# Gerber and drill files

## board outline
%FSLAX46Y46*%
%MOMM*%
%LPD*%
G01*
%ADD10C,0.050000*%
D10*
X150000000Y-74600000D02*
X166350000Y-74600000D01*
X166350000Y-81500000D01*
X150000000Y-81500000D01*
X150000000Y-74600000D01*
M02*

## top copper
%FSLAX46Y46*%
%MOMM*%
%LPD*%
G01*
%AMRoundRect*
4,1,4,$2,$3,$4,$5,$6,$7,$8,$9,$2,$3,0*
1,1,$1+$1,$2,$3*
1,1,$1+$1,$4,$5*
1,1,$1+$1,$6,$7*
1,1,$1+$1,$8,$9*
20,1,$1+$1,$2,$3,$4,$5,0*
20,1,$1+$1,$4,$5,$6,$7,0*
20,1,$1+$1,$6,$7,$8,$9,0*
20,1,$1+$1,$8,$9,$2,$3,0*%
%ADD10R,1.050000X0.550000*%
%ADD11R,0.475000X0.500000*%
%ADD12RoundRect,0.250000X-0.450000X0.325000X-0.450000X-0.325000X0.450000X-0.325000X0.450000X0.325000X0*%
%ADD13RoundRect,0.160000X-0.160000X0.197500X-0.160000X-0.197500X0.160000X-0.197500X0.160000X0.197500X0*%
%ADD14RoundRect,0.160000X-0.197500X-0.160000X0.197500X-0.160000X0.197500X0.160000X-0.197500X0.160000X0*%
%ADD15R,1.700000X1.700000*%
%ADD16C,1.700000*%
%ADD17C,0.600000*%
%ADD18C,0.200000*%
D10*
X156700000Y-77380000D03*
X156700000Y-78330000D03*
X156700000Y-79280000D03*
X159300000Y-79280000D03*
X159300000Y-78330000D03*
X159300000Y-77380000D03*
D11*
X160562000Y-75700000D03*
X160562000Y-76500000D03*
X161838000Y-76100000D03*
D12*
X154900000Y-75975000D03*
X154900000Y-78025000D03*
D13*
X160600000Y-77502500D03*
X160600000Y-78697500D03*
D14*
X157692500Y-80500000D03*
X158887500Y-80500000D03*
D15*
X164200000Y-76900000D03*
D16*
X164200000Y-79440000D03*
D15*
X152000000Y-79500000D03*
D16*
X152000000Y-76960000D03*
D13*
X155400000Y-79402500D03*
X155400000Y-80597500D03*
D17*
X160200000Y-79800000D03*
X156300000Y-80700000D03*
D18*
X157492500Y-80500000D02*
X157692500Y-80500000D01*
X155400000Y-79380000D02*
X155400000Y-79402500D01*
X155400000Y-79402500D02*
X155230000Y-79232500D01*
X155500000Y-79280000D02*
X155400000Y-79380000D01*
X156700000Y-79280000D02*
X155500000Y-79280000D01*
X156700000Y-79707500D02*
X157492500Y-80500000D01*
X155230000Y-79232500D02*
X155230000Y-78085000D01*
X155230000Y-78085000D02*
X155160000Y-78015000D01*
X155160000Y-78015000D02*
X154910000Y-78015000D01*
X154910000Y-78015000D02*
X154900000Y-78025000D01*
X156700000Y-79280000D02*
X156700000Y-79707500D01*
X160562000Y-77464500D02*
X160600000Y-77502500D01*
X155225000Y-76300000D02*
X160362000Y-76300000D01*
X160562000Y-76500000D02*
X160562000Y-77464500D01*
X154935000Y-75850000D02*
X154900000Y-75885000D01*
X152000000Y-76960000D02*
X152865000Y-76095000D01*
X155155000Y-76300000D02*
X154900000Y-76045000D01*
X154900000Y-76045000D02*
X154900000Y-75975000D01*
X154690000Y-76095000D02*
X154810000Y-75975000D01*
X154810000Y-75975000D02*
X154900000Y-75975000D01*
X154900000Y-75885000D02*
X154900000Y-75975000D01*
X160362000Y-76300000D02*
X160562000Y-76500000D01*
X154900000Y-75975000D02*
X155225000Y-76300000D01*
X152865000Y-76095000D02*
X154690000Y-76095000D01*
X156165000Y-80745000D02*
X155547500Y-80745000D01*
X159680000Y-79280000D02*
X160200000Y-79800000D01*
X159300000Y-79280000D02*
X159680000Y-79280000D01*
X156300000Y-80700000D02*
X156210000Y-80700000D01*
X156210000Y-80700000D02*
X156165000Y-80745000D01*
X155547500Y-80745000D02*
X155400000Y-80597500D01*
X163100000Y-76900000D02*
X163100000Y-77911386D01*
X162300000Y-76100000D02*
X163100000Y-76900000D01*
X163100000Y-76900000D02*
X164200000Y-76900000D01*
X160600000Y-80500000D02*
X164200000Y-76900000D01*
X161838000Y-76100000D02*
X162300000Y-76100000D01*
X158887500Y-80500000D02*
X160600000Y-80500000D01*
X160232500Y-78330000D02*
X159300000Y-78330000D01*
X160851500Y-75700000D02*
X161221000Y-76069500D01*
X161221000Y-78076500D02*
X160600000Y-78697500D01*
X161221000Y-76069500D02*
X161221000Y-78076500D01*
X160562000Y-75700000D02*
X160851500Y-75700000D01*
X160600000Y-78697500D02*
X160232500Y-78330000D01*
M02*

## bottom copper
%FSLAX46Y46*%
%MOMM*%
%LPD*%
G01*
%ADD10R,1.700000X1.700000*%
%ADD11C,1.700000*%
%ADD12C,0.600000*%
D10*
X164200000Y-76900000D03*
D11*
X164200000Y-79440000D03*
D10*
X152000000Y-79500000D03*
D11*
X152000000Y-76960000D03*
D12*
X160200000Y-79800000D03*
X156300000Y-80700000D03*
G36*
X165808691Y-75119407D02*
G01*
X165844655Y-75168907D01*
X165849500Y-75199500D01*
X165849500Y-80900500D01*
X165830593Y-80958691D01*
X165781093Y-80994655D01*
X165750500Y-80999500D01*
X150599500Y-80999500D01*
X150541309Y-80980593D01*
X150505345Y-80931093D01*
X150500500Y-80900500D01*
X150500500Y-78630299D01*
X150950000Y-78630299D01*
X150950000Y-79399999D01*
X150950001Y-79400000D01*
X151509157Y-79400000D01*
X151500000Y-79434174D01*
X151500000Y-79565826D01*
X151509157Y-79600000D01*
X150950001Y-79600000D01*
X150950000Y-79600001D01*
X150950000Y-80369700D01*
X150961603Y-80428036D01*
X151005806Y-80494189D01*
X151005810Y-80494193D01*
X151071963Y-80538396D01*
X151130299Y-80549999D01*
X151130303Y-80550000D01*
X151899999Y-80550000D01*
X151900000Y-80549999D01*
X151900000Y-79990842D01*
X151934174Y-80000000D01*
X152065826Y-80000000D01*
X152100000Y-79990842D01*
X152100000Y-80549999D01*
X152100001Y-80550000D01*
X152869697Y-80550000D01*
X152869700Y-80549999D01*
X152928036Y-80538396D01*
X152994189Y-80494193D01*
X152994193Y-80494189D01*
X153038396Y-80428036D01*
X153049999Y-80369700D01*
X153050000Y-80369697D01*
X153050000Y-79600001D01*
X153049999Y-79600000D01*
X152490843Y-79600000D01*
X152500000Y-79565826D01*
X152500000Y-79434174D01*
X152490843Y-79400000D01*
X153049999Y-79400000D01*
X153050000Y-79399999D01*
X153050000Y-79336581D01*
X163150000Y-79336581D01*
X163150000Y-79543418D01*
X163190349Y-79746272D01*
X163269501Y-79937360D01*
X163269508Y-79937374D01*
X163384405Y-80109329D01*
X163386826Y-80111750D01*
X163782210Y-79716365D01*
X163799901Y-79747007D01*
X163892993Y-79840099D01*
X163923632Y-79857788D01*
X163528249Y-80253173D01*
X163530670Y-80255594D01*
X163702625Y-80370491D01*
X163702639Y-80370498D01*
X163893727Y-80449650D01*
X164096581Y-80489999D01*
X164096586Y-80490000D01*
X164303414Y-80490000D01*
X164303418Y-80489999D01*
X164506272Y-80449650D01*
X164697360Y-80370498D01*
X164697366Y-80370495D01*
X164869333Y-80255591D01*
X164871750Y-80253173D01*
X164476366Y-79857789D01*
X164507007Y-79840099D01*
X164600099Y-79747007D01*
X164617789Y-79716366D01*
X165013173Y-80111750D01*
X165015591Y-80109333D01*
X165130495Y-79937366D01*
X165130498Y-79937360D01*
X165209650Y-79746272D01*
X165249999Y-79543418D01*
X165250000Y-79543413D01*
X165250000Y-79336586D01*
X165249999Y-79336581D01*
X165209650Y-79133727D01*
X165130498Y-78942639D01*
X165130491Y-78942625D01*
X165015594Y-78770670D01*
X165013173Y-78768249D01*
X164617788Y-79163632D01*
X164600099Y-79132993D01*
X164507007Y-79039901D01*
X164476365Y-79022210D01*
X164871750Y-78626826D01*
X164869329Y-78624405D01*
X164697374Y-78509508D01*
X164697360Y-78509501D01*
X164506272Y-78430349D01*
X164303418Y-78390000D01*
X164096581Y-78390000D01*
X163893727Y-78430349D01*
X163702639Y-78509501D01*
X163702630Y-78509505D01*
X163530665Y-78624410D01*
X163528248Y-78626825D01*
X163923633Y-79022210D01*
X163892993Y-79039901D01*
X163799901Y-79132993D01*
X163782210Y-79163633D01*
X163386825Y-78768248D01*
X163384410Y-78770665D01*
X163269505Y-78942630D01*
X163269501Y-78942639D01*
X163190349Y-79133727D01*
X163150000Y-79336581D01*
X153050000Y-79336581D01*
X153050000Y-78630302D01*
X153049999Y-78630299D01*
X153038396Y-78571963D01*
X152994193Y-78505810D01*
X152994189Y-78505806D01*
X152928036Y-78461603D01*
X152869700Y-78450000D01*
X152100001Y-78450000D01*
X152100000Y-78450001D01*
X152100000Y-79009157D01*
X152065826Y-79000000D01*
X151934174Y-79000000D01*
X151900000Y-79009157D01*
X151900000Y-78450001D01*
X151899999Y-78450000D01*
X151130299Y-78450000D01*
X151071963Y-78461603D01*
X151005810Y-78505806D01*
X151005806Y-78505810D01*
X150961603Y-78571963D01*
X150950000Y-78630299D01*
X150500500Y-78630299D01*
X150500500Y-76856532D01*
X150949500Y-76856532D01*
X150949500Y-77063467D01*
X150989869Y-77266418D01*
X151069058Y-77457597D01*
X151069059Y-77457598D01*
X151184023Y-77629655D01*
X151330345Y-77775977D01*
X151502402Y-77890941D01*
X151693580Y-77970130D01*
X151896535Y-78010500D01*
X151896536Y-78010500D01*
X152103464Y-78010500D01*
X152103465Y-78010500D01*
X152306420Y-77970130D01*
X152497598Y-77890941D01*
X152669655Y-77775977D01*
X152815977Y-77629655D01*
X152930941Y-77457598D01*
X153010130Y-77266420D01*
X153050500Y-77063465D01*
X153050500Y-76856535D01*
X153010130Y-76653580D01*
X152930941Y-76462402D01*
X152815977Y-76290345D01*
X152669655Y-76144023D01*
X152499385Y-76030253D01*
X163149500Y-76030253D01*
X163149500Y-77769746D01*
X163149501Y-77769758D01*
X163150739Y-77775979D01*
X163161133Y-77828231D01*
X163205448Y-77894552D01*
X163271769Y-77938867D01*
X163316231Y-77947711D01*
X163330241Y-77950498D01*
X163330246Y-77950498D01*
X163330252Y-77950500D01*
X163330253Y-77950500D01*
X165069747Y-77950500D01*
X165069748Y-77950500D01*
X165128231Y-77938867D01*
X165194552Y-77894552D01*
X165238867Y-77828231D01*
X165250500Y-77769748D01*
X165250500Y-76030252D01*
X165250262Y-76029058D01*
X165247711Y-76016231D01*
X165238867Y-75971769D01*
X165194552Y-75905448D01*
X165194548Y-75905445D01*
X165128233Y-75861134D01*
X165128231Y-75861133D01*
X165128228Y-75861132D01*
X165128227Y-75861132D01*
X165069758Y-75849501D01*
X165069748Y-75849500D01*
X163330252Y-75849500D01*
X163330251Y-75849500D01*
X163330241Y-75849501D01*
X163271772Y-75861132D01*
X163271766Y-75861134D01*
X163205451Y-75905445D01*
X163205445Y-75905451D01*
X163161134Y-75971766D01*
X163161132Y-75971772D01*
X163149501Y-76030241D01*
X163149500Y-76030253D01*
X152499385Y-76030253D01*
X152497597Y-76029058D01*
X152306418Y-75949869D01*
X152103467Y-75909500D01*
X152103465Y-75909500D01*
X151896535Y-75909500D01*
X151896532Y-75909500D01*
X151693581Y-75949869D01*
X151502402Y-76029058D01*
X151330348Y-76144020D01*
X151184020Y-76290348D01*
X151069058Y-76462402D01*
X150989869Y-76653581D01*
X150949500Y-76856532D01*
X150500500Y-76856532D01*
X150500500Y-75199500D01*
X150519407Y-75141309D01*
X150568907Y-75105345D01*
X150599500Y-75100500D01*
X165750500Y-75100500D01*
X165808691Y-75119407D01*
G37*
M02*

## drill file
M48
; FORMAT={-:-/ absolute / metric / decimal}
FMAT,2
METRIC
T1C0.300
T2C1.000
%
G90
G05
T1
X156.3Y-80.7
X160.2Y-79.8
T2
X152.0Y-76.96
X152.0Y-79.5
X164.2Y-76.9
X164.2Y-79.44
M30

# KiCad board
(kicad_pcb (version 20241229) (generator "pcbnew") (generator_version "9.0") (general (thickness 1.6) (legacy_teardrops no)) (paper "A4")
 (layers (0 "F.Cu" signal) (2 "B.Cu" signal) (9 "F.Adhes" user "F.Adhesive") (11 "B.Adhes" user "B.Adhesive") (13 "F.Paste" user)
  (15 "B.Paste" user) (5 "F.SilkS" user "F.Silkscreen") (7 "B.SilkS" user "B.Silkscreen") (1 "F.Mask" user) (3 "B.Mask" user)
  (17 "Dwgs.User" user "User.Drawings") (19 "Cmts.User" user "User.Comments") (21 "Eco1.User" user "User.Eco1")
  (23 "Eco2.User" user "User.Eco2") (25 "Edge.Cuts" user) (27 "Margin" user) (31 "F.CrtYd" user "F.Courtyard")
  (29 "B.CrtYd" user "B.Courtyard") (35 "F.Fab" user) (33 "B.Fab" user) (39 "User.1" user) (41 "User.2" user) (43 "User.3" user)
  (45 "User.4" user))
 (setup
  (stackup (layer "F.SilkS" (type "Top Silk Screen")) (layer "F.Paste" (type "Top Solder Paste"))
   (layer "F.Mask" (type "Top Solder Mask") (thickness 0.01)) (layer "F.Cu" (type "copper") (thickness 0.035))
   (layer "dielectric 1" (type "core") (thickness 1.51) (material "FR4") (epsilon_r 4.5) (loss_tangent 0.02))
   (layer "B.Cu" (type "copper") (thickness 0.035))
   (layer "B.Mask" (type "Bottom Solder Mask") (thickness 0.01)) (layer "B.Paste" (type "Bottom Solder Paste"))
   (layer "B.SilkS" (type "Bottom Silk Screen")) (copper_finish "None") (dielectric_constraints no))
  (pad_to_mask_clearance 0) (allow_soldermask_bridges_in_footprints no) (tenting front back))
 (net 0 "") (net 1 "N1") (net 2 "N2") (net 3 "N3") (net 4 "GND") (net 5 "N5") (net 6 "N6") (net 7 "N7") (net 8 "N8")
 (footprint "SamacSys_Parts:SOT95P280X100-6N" (layer "F.Cu") (at 158 78.33)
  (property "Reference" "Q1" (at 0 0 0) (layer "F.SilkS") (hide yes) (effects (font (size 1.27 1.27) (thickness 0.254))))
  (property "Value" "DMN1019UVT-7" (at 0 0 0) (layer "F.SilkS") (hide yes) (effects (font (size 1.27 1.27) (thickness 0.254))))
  (pad "1" smd rect (at -1.3 -0.95 90) (size 0.55 1.05) (layers "F.Cu" "F.Mask" "F.Paste") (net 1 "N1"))
  (pad "2" smd rect (at -1.3 0 90) (size 0.55 1.05) (layers "F.Cu" "F.Mask" "F.Paste") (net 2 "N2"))
  (pad "3" smd rect (at -1.3 0.95 90) (size 0.55 1.05) (layers "F.Cu" "F.Mask" "F.Paste") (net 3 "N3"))
  (pad "4" smd rect (at 1.3 0.95 90) (size 0.55 1.05) (layers "F.Cu" "F.Mask" "F.Paste") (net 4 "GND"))
  (pad "5" smd rect (at 1.3 0 90) (size 0.55 1.05) (layers "F.Cu" "F.Mask" "F.Paste") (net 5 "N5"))
  (pad "6" smd rect (at 1.3 -0.95 90) (size 0.55 1.05) (layers "F.Cu" "F.Mask" "F.Paste") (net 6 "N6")))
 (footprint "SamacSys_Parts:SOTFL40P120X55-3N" (layer "F.Cu") (at 161.2 76.1)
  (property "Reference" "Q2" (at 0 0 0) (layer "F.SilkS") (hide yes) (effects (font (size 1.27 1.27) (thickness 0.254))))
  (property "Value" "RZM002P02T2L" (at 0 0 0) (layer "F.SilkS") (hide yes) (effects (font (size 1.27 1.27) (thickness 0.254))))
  (pad "1" smd rect (at -0.638 -0.4) (size 0.475 0.5) (layers "F.Cu" "F.Mask" "F.Paste") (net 5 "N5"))
  (pad "2" smd rect (at -0.638 0.4) (size 0.475 0.5) (layers "F.Cu" "F.Mask" "F.Paste") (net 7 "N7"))
  (pad "3" smd rect (at 0.638 0) (size 0.475 0.5) (layers "F.Cu" "F.Mask" "F.Paste") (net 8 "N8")))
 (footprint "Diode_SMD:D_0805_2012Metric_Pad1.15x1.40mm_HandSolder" (layer "F.Cu") (at 154.9 77 -90)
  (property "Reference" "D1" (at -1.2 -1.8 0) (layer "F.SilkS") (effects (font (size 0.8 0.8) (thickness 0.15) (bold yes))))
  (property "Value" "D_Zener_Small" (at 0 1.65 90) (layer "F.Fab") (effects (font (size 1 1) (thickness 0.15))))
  (pad "1" smd roundrect (at -1.025 0 270) (size 1.15 1.4) (layers "F.Cu" "F.Mask" "F.Paste") (roundrect_rratio 0.217391) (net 7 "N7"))
  (pad "2" smd roundrect (at 1.025 0 270) (size 1.15 1.4) (layers "F.Cu" "F.Mask" "F.Paste") (roundrect_rratio 0.217391) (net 3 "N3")))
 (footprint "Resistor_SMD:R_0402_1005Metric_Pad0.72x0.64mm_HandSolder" (layer "F.Cu") (at 160.6 78.1 -90)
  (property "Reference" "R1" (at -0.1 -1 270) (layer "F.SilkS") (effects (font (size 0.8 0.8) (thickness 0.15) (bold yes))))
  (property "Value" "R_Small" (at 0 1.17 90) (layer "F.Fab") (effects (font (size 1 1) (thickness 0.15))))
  (pad "1" smd roundrect (at -0.5975 0 270) (size 0.715 0.64) (layers "F.Cu" "F.Mask" "F.Paste") (roundrect_rratio 0.25) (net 7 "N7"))
  (pad "2" smd roundrect (at 0.5975 0 270) (size 0.715 0.64) (layers "F.Cu" "F.Mask" "F.Paste") (roundrect_rratio 0.25) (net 5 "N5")))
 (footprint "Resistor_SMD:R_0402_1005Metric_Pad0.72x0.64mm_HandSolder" (layer "F.Cu") (at 158.29 80.5)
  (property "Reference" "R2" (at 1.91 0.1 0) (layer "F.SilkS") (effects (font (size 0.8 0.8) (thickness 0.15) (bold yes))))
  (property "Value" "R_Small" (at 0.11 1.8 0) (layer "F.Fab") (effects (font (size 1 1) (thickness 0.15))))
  (pad "1" smd roundrect (at -0.5975 0) (size 0.715 0.64) (layers "F.Cu" "F.Mask" "F.Paste") (roundrect_rratio 0.25) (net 3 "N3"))
  (pad "2" smd roundrect (at 0.5975 0) (size 0.715 0.64) (layers "F.Cu" "F.Mask" "F.Paste") (roundrect_rratio 0.25) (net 8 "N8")))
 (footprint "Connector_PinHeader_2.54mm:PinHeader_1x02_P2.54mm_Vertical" (layer "F.Cu") (at 164.2 76.9)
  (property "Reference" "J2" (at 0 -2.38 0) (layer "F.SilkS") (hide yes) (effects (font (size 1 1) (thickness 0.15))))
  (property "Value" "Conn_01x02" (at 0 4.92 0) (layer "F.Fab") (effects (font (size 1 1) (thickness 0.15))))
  (pad "1" thru_hole rect (at 0 0) (size 1.7 1.7) (drill 1) (layers "*.Cu" "*.Mask") (remove_unused_layers no) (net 8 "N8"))
  (pad "2" thru_hole circle (at 0 2.54) (size 1.7 1.7) (drill 1) (layers "*.Cu" "*.Mask") (remove_unused_layers no) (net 4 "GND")))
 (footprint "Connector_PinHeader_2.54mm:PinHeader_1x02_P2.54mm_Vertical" (layer "F.Cu") (at 152 79.5 180)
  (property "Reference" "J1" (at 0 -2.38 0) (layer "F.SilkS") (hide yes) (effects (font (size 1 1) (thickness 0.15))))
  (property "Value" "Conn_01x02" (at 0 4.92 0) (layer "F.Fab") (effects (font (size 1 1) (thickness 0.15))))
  (pad "1" thru_hole rect (at 0 0 180) (size 1.7 1.7) (drill 1) (layers "*.Cu" "*.Mask") (remove_unused_layers no) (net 4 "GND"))
  (pad "2" thru_hole circle (at 0 2.54 180) (size 1.7 1.7) (drill 1) (layers "*.Cu" "*.Mask") (remove_unused_layers no) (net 7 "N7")))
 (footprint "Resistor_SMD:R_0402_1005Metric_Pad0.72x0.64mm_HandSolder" (layer "F.Cu") (at 155.4 80 -90)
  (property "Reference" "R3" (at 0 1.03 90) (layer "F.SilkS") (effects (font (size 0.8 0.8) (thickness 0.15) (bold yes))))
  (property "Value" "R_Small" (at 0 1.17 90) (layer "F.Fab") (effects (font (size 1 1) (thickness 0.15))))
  (pad "1" smd roundrect (at -0.5975 0 270) (size 0.715 0.64) (layers "F.Cu" "F.Mask" "F.Paste") (roundrect_rratio 0.25) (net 3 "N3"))
  (pad "2" smd roundrect (at 0.5975 0 270) (size 0.715 0.64) (layers "F.Cu" "F.Mask" "F.Paste") (roundrect_rratio 0.25) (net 4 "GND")))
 (gr_rect (start 150 74.6) (end 166.35 81.5) (stroke (width 0.05) (type default)) (fill no) (layer "Edge.Cuts"))
 (segment (start 157.4925 80.5) (end 157.6925 80.5) (width 0.2) (layer "F.Cu") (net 3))
 (segment (start 155.4 79.38) (end 155.4 79.4025) (width 0.2) (layer "F.Cu") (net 3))
 (segment (start 155.4 79.4025) (end 155.23 79.2325) (width 0.2) (layer "F.Cu") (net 3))
 (segment (start 155.5 79.28) (end 155.4 79.38) (width 0.2) (layer "F.Cu") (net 3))
 (segment (start 156.7 79.28) (end 155.5 79.28) (width 0.2) (layer "F.Cu") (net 3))
 (segment (start 156.7 79.7075) (end 157.4925 80.5) (width 0.2) (layer "F.Cu") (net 3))
 (segment (start 155.23 79.2325) (end 155.23 78.085) (width 0.2) (layer "F.Cu") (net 3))
 (segment (start 155.23 78.085) (end 155.16 78.015) (width 0.2) (layer "F.Cu") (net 3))
 (segment (start 155.16 78.015) (end 154.91 78.015) (width 0.2) (layer "F.Cu") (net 3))
 (segment (start 154.91 78.015) (end 154.9 78.025) (width 0.2) (layer "F.Cu") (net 3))
 (segment (start 156.7 79.28) (end 156.7 79.7075) (width 0.2) (layer "F.Cu") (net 3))
 (segment (start 160.562 77.4645) (end 160.6 77.5025) (width 0.2) (layer "F.Cu") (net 7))
 (segment (start 155.225 76.3) (end 160.362 76.3) (width 0.2) (layer "F.Cu") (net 7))
 (segment (start 160.562 76.5) (end 160.562 77.4645) (width 0.2) (layer "F.Cu") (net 7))
 (segment (start 154.935 75.85) (end 154.9 75.885) (width 0.2) (layer "F.Cu") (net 7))
 (segment (start 152 76.96) (end 152.865 76.095) (width 0.2) (layer "F.Cu") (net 7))
 (segment (start 155.155 76.3) (end 154.9 76.045) (width 0.2) (layer "F.Cu") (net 7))
 (segment (start 154.9 76.045) (end 154.9 75.975) (width 0.2) (layer "F.Cu") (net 7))
 (segment (start 154.69 76.095) (end 154.81 75.975) (width 0.2) (layer "F.Cu") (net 7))
 (segment (start 154.81 75.975) (end 154.9 75.975) (width 0.2) (layer "F.Cu") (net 7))
 (segment (start 154.9 75.885) (end 154.9 75.975) (width 0.2) (layer "F.Cu") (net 7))
 (segment (start 160.362 76.3) (end 160.562 76.5) (width 0.2) (layer "F.Cu") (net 7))
 (segment (start 154.9 75.975) (end 155.225 76.3) (width 0.2) (layer "F.Cu") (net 7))
 (segment (start 152.865 76.095) (end 154.69 76.095) (width 0.2) (layer "F.Cu") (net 7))
 (segment (start 156.165 80.745) (end 155.5475 80.745) (width 0.2) (layer "F.Cu") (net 4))
 (segment (start 159.68 79.28) (end 160.2 79.8) (width 0.2) (layer "F.Cu") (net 4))
 (segment (start 159.3 79.28) (end 159.68 79.28) (width 0.2) (layer "F.Cu") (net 4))
 (segment (start 156.3 80.7) (end 156.21 80.7) (width 0.2) (layer "F.Cu") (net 4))
 (segment (start 156.21 80.7) (end 156.165 80.745) (width 0.2) (layer "F.Cu") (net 4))
 (segment (start 155.5475 80.745) (end 155.4 80.5975) (width 0.2) (layer "F.Cu") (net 4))
 (via (at 160.2 79.8) (size 0.6) (drill 0.3) (layers "F.Cu" "B.Cu") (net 4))
 (via (at 156.3 80.7) (size 0.6) (drill 0.3) (layers "F.Cu" "B.Cu") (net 4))
 (segment (start 163.1 76.9) (end 163.1 77.911386) (width 0.2) (layer "F.Cu") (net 8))
 (segment (start 162.3 76.1) (end 163.1 76.9) (width 0.2) (layer "F.Cu") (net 8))
 (segment (start 163.1 76.9) (end 164.2 76.9) (width 0.2) (layer "F.Cu") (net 8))
 (segment (start 160.6 80.5) (end 164.2 76.9) (width 0.2) (layer "F.Cu") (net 8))
 (segment (start 161.838 76.1) (end 162.3 76.1) (width 0.2) (layer "F.Cu") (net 8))
 (segment (start 158.8875 80.5) (end 160.6 80.5) (width 0.2) (layer "F.Cu") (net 8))
 (segment (start 160.2325 78.33) (end 159.3 78.33) (width 0.2) (layer "F.Cu") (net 5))
 (segment (start 160.8515 75.7) (end 161.221 76.0695) (width 0.2) (layer "F.Cu") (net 5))
 (segment (start 161.221 78.0765) (end 160.6 78.6975) (width 0.2) (layer "F.Cu") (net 5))
 (segment (start 161.221 76.0695) (end 161.221 78.0765) (width 0.2) (layer "F.Cu") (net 5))
 (segment (start 160.562 75.7) (end 160.8515 75.7) (width 0.2) (layer "F.Cu") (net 5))
 (segment (start 160.6 78.6975) (end 160.2325 78.33) (width 0.2) (layer "F.Cu") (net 5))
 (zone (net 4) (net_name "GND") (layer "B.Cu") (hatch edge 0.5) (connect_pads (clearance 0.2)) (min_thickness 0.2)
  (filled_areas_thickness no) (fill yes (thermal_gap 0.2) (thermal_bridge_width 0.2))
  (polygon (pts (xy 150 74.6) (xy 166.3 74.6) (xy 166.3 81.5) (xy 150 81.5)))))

